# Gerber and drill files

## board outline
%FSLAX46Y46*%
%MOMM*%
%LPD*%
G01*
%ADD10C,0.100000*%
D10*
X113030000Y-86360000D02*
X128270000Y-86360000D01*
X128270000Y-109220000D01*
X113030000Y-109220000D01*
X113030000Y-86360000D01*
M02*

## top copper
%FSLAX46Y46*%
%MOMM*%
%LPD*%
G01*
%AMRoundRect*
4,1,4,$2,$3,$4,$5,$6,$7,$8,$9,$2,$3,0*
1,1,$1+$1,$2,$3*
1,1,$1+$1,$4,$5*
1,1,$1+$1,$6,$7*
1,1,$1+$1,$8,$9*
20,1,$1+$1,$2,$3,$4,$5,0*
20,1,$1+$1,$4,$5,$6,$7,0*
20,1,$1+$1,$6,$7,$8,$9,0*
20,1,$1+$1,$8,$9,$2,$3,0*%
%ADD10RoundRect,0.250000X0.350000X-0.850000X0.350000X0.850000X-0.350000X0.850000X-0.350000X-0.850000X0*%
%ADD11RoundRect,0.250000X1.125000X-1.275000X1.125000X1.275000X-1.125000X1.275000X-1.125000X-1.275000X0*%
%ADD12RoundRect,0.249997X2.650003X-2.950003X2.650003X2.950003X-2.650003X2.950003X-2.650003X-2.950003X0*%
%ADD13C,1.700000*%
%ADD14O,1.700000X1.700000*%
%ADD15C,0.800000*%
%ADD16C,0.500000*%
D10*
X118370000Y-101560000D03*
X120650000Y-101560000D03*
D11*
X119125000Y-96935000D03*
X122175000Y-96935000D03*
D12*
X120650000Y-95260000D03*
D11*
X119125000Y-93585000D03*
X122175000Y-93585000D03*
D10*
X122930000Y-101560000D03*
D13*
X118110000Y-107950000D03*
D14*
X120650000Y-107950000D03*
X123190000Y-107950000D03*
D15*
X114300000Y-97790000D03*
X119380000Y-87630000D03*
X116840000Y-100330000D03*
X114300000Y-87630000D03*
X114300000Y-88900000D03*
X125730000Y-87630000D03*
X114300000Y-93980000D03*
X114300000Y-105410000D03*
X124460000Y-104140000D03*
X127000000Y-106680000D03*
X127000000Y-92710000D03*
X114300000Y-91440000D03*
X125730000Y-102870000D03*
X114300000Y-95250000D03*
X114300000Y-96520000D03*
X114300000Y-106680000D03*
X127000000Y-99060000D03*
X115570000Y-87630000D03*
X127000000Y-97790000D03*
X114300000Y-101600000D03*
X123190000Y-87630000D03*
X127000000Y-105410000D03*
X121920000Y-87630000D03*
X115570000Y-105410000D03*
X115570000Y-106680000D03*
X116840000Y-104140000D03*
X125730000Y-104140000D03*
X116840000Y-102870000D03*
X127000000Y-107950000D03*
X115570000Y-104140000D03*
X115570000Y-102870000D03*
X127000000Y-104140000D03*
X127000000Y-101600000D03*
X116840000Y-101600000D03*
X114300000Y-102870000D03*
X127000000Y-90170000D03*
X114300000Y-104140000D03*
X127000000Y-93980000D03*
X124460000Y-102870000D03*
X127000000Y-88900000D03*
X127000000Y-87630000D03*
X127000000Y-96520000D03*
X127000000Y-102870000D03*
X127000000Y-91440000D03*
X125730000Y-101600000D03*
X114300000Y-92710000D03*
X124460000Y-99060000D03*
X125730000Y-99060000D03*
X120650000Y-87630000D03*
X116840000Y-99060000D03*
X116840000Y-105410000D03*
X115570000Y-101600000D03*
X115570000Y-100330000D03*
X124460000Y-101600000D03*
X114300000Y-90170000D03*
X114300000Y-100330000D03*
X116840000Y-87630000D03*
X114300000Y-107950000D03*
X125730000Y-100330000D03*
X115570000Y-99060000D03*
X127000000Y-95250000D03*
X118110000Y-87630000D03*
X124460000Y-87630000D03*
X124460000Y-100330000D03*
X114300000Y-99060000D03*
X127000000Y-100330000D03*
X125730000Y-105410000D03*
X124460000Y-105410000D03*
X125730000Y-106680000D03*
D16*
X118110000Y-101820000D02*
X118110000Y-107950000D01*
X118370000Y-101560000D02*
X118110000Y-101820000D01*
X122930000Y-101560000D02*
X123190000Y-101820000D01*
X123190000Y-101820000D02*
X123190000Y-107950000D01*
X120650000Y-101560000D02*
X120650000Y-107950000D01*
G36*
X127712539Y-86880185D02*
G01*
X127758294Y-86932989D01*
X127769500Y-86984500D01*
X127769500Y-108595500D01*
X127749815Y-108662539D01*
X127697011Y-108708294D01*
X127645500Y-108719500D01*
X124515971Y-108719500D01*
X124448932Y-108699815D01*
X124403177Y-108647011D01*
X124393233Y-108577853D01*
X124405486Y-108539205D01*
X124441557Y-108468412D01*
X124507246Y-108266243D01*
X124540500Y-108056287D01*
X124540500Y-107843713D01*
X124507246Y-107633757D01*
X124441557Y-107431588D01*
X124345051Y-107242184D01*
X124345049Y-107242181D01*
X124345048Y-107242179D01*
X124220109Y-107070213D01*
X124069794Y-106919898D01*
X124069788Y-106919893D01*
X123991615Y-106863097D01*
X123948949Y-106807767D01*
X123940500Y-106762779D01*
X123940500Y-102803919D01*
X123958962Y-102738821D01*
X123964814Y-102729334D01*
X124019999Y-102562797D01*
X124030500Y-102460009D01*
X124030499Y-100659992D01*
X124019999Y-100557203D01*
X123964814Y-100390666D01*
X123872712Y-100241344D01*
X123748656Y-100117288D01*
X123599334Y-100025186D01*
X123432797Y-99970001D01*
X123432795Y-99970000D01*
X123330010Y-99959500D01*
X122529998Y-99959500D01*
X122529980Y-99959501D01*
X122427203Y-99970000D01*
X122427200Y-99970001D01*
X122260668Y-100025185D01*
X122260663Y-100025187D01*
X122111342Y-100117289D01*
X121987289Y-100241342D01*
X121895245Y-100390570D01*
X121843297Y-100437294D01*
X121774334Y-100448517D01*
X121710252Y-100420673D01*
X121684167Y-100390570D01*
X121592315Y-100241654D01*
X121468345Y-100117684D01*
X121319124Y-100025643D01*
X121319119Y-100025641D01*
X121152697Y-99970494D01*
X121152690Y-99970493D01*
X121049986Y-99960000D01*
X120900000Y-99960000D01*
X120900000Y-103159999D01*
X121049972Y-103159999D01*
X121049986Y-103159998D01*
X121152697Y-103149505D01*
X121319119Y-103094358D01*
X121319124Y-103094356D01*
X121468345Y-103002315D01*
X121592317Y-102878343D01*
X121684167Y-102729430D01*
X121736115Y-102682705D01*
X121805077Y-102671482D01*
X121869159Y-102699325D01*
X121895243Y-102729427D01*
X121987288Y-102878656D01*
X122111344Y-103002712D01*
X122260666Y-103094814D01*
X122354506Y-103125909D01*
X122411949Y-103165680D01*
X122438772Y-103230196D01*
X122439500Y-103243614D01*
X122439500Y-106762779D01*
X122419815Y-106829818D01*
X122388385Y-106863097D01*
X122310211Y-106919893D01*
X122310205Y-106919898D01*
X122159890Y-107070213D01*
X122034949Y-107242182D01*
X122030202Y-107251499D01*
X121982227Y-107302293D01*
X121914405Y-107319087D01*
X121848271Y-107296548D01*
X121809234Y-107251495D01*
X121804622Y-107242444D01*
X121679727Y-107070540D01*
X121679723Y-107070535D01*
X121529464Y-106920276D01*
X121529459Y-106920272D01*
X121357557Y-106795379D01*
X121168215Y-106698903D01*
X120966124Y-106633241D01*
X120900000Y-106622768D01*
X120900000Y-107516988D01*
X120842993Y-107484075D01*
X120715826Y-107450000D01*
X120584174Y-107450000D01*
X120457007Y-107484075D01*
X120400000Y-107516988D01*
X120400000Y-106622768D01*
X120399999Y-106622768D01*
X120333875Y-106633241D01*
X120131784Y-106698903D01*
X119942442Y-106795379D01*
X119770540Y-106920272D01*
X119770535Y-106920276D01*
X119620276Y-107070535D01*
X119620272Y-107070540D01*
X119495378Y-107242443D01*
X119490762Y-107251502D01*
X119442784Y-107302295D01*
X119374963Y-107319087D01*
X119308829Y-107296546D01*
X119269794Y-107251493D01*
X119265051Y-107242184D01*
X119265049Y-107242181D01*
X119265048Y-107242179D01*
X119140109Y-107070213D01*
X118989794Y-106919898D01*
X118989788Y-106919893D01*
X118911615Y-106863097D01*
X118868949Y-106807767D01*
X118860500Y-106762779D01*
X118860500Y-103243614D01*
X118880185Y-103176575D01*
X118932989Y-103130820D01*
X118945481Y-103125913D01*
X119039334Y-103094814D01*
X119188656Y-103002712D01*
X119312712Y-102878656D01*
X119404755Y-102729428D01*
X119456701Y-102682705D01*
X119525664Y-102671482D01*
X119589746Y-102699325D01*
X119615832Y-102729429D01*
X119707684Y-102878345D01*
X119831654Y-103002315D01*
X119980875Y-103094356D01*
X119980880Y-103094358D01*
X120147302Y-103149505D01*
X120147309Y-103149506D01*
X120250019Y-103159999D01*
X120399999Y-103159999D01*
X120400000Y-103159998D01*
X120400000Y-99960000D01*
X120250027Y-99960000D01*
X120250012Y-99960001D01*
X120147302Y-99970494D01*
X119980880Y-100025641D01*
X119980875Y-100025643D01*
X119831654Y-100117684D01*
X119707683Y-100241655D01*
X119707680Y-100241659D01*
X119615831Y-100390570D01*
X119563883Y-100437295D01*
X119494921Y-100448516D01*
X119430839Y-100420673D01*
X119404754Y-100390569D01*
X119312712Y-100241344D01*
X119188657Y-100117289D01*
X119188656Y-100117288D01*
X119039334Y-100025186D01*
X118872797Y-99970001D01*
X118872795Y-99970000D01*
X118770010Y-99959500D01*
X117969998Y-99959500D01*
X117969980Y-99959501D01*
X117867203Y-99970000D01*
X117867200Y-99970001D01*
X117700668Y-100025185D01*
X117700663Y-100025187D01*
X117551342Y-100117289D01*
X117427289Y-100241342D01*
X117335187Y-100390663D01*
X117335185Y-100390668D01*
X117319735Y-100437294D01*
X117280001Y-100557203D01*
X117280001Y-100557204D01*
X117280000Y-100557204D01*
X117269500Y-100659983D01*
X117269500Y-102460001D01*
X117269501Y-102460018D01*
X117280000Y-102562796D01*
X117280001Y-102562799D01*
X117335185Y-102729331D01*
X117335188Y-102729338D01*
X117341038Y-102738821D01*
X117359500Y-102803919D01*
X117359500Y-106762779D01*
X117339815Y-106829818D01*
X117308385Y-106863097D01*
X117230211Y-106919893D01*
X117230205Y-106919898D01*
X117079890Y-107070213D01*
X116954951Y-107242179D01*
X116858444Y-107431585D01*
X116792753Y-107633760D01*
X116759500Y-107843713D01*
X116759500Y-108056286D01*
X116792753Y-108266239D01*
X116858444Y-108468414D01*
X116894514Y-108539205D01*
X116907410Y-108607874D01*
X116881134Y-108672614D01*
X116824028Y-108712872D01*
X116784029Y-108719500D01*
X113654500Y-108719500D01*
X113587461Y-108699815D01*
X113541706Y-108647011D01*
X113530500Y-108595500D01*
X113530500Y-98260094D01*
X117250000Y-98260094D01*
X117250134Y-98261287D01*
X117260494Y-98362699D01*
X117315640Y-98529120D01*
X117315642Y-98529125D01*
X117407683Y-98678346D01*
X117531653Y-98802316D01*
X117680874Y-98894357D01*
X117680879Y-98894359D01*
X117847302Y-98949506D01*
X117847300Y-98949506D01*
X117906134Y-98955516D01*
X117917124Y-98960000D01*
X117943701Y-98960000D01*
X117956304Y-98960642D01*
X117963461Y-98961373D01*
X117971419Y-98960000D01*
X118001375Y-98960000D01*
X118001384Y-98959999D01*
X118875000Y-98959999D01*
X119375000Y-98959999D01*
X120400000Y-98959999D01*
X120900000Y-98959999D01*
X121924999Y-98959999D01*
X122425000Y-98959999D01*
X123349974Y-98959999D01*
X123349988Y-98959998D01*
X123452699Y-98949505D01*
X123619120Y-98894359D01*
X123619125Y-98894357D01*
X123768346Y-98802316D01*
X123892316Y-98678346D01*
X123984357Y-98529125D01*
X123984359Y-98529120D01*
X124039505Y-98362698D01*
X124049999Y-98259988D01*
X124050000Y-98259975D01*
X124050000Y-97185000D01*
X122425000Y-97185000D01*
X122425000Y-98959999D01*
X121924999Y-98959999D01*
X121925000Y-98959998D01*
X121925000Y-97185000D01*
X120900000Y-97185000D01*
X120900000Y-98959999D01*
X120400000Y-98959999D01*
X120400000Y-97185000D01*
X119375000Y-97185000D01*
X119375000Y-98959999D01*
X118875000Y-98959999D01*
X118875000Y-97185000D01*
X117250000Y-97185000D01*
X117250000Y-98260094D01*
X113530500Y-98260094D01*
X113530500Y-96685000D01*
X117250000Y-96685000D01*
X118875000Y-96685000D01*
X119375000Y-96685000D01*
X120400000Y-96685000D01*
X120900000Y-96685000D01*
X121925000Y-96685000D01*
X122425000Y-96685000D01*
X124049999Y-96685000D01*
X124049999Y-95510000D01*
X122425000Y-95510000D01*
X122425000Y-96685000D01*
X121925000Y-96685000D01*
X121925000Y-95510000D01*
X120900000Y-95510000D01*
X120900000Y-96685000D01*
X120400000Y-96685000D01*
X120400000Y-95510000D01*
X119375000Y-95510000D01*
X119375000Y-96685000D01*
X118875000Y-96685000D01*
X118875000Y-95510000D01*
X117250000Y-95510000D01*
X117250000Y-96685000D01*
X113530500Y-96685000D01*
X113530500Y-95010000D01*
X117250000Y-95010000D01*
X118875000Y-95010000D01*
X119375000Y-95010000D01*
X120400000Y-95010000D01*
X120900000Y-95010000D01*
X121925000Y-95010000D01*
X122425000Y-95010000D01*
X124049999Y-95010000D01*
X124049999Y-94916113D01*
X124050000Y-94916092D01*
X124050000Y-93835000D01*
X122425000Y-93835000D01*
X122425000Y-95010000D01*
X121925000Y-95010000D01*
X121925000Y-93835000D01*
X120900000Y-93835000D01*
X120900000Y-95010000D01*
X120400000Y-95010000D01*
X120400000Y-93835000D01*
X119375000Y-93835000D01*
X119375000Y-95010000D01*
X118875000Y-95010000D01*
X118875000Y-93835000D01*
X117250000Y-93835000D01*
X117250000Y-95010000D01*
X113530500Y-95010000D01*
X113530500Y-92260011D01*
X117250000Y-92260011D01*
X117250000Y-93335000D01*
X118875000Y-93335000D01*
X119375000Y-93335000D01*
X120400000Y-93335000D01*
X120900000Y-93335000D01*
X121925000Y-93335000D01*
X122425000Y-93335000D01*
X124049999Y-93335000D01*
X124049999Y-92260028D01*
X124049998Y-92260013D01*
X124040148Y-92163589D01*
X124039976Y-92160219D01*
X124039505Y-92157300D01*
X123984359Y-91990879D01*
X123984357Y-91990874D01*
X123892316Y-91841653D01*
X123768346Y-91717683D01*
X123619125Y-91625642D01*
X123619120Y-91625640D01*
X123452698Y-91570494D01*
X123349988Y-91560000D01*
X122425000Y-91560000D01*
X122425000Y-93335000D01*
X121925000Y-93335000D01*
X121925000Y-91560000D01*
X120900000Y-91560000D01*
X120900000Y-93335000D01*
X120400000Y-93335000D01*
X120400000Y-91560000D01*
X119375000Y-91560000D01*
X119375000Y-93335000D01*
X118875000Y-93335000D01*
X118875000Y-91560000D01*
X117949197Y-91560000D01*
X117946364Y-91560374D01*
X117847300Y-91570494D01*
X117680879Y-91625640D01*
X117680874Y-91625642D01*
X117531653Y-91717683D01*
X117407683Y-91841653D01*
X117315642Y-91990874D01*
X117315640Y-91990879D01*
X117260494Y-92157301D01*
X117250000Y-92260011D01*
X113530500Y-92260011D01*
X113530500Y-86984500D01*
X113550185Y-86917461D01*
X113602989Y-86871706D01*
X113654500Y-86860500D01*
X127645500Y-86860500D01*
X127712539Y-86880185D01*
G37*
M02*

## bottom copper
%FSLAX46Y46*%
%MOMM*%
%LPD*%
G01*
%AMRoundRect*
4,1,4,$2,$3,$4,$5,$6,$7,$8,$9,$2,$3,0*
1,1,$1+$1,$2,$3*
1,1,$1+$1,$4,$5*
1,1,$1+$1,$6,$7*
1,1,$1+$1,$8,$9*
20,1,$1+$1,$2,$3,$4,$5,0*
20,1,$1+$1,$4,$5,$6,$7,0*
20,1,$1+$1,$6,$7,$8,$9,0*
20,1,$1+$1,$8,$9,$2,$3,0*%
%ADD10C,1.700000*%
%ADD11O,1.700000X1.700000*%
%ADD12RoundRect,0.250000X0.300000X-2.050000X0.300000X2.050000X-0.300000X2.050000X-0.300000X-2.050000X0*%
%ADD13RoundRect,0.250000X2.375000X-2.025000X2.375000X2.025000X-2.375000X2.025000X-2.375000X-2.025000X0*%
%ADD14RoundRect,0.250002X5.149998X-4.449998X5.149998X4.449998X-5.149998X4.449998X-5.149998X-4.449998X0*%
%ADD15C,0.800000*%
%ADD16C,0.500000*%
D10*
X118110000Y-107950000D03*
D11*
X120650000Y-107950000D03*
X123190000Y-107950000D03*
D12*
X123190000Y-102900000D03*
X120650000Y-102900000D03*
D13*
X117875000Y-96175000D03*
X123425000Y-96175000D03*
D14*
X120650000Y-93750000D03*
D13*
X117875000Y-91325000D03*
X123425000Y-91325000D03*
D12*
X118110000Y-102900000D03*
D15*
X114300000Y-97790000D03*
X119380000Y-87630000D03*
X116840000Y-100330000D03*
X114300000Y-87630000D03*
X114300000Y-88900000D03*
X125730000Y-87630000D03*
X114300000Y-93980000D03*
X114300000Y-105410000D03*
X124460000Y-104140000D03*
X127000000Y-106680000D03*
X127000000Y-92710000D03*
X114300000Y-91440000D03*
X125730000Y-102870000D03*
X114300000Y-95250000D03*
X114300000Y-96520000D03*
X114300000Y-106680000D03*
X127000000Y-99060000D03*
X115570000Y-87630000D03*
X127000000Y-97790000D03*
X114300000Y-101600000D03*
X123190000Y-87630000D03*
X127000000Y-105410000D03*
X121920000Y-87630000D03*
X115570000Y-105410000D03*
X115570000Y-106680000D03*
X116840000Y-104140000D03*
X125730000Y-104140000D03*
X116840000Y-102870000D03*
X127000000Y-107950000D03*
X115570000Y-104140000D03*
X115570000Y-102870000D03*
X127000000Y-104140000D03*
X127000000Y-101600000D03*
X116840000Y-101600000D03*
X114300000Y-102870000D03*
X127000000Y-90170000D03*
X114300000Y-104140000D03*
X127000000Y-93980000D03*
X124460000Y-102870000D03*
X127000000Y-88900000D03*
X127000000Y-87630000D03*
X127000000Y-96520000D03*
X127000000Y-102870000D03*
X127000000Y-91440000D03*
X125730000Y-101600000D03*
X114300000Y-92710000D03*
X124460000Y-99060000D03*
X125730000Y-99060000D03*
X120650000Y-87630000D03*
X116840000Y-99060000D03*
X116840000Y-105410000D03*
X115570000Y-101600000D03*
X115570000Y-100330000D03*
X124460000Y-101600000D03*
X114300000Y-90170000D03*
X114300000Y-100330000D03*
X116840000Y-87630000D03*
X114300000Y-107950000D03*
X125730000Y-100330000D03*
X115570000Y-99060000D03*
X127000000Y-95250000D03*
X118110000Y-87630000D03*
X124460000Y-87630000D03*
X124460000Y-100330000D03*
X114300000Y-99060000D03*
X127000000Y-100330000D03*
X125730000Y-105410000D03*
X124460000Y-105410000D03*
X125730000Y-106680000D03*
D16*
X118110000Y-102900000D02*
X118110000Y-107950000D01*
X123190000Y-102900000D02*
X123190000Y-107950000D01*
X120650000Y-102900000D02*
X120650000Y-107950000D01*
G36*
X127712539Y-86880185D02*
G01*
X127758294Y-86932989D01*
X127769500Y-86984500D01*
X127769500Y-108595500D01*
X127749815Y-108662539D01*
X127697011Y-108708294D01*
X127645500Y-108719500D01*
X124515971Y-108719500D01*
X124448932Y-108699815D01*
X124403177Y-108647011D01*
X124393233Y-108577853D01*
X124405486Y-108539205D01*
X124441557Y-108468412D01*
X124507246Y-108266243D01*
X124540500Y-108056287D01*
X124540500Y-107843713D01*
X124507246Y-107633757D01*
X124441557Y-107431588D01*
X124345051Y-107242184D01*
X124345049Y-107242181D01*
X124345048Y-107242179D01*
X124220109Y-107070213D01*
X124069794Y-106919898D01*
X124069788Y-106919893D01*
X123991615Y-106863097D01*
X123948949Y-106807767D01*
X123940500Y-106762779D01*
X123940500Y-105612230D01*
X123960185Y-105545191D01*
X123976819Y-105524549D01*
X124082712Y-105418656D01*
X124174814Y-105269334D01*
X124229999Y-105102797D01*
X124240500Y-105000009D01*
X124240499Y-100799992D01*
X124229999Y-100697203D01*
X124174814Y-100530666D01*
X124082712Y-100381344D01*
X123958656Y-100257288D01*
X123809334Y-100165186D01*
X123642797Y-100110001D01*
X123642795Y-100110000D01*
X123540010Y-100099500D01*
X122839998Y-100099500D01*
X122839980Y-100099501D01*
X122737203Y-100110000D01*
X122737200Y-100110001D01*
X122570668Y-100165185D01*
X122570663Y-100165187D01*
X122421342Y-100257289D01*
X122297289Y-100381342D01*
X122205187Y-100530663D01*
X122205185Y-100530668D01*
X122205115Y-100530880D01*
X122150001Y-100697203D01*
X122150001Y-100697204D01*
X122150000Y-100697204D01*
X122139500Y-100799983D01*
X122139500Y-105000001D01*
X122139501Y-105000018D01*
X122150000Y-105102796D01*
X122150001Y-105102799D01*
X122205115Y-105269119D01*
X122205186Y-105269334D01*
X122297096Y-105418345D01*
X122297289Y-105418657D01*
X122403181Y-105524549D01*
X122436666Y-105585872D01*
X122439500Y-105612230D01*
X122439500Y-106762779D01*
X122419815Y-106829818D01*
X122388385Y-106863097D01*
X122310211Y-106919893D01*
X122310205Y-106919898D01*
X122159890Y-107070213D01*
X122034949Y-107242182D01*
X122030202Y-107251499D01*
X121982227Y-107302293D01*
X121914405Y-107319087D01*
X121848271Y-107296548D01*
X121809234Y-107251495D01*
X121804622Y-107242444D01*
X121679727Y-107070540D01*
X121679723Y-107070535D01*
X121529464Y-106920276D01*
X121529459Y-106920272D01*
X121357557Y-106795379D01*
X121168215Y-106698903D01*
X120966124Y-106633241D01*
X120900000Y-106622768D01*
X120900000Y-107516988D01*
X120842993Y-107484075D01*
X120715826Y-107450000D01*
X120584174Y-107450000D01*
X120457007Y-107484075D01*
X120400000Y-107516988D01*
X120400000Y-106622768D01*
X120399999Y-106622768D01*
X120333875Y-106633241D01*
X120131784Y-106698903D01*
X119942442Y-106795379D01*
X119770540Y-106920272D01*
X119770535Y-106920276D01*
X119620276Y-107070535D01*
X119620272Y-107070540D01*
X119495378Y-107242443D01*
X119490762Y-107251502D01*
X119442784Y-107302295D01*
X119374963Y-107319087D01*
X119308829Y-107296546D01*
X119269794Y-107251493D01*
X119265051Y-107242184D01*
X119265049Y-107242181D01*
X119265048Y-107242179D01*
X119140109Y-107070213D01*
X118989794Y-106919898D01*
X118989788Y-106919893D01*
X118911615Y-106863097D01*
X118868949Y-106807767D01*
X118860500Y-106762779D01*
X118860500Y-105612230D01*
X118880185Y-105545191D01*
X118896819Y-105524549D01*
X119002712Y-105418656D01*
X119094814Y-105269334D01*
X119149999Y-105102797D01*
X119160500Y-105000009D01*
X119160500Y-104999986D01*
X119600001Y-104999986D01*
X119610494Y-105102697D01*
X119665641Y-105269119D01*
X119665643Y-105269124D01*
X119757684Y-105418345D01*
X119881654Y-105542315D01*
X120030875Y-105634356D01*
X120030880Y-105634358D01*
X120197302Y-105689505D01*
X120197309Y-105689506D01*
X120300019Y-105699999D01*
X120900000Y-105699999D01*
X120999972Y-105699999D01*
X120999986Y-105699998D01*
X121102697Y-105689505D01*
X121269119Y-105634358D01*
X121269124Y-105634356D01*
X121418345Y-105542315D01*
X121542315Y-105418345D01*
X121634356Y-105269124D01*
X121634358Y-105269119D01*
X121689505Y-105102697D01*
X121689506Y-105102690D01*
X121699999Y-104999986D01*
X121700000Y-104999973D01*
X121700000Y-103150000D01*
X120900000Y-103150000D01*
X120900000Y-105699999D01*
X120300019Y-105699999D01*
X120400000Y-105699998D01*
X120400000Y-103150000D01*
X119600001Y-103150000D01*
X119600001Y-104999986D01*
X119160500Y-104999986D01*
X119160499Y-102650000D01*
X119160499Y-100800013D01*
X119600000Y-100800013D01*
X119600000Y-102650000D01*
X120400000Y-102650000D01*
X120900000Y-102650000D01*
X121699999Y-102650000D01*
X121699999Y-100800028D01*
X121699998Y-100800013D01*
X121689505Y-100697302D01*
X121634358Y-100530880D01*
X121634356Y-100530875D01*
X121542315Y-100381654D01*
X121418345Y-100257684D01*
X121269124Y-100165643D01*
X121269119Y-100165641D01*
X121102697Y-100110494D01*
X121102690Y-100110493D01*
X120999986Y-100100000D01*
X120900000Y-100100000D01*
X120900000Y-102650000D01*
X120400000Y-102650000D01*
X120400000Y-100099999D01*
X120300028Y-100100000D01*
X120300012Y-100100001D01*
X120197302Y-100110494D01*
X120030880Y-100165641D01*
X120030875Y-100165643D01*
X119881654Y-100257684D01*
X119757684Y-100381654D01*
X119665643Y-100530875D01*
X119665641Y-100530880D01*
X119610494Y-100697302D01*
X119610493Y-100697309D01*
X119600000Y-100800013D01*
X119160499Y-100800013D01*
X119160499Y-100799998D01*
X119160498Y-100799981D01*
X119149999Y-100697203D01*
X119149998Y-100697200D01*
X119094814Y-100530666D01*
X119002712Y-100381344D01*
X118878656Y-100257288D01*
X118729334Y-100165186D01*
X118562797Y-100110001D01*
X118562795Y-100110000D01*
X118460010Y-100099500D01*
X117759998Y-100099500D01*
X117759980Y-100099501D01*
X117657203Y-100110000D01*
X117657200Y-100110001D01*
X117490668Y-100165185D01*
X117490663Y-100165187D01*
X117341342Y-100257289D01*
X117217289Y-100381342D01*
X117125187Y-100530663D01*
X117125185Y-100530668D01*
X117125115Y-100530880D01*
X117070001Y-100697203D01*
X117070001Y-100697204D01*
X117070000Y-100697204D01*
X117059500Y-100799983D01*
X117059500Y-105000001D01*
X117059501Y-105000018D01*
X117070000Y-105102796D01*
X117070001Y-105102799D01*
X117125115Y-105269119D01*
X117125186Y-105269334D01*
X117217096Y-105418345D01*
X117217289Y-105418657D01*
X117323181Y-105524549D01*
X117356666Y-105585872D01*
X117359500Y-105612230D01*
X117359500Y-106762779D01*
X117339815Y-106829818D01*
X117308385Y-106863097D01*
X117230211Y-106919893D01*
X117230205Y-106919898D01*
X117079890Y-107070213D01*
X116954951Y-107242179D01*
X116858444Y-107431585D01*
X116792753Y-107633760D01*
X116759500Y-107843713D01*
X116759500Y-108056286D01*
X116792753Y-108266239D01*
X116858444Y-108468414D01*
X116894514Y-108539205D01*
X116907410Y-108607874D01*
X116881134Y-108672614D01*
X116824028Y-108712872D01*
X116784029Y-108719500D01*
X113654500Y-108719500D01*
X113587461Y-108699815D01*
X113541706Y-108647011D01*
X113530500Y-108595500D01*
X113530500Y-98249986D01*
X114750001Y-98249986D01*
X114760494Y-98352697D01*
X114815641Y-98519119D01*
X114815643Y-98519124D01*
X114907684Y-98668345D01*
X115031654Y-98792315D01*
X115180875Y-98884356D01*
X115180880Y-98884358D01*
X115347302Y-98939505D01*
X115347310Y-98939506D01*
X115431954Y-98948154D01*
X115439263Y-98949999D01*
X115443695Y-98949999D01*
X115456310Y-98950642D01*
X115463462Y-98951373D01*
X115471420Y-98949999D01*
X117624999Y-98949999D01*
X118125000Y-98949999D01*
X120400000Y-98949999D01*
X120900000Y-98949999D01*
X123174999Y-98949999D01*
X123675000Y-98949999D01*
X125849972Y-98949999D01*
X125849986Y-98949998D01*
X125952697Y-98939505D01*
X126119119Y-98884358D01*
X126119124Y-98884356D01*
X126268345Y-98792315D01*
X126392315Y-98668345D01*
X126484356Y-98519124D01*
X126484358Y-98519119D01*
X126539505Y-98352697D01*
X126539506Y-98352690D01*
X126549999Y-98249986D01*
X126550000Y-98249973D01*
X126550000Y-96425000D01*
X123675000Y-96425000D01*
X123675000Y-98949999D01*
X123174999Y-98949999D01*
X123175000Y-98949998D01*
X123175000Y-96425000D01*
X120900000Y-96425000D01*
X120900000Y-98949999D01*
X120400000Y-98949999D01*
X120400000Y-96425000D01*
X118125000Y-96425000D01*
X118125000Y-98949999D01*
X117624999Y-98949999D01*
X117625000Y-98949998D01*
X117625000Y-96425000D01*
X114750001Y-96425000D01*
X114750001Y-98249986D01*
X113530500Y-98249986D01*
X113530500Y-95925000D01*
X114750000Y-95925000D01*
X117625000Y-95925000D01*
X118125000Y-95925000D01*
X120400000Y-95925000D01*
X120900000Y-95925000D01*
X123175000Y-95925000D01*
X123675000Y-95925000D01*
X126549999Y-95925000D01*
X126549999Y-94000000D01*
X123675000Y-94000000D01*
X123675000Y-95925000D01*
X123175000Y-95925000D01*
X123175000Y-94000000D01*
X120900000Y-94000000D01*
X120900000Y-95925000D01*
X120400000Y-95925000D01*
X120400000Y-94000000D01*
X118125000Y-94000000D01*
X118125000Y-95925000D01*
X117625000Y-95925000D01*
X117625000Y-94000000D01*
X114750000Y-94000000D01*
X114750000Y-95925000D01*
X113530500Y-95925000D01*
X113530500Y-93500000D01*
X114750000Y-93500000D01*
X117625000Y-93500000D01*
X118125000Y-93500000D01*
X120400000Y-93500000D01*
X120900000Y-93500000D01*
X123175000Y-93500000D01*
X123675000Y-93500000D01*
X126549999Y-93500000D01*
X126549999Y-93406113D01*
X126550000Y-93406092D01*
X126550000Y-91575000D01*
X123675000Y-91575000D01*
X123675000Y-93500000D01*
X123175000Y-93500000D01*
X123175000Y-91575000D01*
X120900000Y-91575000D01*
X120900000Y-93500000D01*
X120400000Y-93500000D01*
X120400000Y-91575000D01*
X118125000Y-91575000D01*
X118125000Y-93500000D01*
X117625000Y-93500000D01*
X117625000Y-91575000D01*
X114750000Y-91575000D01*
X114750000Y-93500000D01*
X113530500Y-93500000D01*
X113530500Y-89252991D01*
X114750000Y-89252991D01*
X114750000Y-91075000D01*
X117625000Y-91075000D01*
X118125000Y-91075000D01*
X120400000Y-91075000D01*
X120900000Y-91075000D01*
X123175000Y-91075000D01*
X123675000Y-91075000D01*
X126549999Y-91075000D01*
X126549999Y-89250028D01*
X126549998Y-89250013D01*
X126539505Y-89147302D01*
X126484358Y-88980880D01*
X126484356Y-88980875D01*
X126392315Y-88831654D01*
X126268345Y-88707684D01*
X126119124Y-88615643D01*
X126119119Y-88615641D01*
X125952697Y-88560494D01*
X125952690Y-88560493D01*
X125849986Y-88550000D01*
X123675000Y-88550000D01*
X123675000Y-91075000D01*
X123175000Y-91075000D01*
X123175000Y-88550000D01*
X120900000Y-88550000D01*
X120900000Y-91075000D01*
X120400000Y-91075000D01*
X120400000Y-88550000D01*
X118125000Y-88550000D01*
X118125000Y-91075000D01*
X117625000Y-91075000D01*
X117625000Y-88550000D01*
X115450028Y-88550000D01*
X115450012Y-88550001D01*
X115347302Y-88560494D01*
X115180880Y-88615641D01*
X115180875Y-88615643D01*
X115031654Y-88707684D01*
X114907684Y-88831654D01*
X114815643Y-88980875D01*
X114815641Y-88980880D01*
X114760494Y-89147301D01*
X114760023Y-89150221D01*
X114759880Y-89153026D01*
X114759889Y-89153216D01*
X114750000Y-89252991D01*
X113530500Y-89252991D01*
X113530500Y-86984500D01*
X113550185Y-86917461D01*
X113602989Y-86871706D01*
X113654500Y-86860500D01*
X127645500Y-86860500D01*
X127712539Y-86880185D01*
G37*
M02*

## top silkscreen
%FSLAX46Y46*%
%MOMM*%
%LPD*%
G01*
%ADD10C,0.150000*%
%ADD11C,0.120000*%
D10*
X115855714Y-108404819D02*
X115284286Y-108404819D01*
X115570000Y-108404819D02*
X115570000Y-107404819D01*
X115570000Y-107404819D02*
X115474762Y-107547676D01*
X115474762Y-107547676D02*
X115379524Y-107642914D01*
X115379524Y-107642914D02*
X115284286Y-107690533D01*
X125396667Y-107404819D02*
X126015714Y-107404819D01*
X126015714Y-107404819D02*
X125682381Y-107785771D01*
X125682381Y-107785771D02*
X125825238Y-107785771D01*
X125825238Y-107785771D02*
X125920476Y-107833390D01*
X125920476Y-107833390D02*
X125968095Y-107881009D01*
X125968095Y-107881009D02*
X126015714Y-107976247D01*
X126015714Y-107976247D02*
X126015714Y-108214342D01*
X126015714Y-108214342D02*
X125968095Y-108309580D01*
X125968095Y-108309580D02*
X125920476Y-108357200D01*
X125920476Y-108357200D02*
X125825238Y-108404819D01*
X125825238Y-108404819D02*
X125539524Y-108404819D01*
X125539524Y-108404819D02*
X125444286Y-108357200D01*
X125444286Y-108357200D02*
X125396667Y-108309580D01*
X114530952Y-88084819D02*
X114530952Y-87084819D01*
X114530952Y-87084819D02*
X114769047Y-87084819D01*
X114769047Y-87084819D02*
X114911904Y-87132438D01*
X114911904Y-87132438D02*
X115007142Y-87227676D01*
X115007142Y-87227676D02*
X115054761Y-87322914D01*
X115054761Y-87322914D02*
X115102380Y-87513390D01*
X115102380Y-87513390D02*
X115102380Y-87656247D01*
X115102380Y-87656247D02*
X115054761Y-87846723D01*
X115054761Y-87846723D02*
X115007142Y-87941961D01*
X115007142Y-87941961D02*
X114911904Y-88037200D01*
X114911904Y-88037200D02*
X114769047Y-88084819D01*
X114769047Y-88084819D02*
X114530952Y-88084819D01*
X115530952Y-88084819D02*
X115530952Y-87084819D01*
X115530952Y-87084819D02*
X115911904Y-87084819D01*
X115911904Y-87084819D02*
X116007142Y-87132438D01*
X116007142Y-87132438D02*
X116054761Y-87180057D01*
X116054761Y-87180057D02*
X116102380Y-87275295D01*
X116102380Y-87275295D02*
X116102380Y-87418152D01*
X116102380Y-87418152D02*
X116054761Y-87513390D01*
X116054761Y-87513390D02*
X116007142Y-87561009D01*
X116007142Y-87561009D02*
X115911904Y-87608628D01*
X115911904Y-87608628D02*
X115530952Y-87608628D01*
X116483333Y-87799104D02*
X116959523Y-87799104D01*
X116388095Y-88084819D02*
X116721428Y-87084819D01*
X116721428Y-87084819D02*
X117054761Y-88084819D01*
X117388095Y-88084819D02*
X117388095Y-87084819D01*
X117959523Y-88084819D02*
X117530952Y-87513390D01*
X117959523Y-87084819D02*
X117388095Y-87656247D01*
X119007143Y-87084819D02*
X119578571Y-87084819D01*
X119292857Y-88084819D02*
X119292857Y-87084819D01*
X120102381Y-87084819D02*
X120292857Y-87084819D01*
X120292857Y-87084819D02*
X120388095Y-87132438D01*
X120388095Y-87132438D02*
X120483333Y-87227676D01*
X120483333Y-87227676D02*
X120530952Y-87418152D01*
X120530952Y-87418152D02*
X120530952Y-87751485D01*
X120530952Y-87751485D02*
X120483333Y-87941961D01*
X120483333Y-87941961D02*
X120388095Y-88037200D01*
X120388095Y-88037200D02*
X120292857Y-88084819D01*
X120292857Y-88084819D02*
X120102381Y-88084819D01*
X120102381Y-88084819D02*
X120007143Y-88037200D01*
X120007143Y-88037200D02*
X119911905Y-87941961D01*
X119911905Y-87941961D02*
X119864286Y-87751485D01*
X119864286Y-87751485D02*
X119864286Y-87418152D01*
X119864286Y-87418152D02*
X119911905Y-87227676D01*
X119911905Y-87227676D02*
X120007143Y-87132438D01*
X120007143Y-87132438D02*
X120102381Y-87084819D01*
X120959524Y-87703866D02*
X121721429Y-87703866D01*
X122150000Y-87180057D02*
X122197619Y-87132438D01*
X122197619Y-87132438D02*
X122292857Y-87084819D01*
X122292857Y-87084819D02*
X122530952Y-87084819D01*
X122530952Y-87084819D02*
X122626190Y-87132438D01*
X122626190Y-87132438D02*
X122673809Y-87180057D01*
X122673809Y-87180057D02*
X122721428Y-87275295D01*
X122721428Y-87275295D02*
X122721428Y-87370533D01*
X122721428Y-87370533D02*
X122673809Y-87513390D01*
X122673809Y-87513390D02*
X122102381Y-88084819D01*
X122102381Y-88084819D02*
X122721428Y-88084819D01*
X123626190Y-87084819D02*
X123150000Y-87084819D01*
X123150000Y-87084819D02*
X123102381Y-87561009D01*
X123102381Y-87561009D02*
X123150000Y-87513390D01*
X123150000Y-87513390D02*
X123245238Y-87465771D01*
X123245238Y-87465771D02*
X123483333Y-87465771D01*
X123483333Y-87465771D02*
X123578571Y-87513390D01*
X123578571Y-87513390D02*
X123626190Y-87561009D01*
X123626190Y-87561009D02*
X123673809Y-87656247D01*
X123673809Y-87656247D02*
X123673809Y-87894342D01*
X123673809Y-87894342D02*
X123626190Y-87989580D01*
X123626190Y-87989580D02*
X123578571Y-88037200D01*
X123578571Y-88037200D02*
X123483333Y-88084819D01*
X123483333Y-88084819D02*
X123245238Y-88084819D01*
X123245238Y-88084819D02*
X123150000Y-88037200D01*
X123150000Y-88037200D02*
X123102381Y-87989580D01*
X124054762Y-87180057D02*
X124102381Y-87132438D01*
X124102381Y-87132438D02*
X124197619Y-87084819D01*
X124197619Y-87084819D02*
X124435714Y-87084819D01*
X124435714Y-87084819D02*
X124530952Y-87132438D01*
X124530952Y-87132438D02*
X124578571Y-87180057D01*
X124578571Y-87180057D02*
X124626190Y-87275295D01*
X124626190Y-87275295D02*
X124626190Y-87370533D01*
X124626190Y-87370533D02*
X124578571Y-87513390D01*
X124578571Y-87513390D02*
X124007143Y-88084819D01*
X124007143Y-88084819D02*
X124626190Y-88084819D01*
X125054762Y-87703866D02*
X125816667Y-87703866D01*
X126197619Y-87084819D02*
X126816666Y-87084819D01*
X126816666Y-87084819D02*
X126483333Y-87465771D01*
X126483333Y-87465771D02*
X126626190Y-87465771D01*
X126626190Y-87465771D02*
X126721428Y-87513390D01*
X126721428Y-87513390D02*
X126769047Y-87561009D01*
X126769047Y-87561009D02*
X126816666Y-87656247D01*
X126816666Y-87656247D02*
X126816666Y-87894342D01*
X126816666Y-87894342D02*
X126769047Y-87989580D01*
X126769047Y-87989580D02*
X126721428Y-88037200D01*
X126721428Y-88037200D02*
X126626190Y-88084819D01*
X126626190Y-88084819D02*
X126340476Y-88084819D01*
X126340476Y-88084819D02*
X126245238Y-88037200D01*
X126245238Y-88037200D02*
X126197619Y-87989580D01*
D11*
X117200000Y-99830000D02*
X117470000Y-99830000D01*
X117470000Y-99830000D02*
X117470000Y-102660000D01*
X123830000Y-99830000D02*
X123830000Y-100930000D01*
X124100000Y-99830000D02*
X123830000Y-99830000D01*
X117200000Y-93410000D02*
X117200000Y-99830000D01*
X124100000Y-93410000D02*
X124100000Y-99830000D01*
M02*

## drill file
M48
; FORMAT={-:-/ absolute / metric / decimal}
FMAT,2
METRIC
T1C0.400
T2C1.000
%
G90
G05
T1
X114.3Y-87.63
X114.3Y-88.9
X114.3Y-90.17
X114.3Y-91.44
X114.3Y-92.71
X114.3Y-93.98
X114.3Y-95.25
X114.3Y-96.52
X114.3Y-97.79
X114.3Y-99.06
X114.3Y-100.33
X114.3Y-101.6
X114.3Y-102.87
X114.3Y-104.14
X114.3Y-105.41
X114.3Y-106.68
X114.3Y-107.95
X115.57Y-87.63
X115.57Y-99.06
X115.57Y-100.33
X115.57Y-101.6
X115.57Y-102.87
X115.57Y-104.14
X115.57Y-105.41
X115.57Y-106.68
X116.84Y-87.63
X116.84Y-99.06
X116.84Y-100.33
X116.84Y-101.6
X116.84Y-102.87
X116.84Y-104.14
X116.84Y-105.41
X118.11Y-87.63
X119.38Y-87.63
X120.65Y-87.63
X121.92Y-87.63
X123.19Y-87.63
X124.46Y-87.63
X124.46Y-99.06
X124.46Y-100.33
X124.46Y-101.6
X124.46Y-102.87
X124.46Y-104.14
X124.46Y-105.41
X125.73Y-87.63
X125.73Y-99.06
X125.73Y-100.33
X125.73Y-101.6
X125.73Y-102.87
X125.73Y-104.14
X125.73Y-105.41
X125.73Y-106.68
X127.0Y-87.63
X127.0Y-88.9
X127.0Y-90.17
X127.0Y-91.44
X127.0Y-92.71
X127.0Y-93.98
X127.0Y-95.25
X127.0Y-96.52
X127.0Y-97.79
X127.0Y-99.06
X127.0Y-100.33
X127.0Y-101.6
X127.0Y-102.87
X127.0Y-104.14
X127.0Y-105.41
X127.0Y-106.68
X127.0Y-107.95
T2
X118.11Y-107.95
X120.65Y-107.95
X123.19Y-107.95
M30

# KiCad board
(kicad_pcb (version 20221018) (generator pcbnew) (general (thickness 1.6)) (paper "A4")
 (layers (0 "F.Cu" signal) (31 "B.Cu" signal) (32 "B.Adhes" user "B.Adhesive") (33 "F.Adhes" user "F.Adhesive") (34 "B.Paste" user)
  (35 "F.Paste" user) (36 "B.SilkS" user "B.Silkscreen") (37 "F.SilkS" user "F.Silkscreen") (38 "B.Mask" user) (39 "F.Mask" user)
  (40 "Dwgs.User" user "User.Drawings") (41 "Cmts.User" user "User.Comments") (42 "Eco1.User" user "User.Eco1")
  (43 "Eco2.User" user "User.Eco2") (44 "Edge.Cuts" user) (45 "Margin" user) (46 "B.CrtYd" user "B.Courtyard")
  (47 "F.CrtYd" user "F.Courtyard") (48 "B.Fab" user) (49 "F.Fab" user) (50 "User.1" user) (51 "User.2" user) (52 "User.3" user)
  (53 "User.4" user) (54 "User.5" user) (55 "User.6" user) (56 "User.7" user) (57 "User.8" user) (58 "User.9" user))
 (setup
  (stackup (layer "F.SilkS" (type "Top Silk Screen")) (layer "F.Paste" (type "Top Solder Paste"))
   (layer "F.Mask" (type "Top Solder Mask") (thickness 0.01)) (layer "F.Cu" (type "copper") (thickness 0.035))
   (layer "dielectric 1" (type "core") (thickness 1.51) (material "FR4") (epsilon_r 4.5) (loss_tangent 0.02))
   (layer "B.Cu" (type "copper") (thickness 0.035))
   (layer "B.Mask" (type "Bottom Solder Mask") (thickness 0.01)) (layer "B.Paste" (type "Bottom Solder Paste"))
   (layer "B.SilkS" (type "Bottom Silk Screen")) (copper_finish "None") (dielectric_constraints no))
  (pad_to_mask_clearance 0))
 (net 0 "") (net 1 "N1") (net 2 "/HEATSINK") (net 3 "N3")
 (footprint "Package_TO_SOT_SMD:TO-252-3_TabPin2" (layer "F.Cu") (at 120.65 96.52 90)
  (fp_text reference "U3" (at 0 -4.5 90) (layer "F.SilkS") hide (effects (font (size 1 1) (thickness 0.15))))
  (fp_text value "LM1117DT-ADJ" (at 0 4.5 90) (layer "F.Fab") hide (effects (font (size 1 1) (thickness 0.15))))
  (fp_line (start -3.31 -3.45) (end -3.31 -3.18) (stroke (width 0.12) (type solid)) (layer "F.SilkS"))
  (fp_line (start -3.31 -3.18) (end -6.14 -3.18) (stroke (width 0.12) (type solid)) (layer "F.SilkS"))
  (fp_line (start -3.31 3.18) (end -4.41 3.18) (stroke (width 0.12) (type solid)) (layer "F.SilkS"))
  (fp_line (start -3.31 3.45) (end -3.31 3.18) (stroke (width 0.12) (type solid)) (layer "F.SilkS"))
  (fp_line (start 3.11 -3.45) (end -3.31 -3.45) (stroke (width 0.12) (type solid)) (layer "F.SilkS"))
  (fp_line (start 3.11 3.45) (end -3.31 3.45) (stroke (width 0.12) (type solid)) (layer "F.SilkS"))
  (pad "1" smd roundrect (at -5.04 -2.28 90) (size 2.2 1.2) (layers "F.Cu" "F.Paste" "F.Mask") (roundrect_rratio 0.208333) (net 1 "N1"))
  (pad "2" smd roundrect (at -5.04 0 90) (size 2.2 1.2) (layers "F.Cu" "F.Paste" "F.Mask") (roundrect_rratio 0.208333) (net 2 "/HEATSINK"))
  (pad "2" smd roundrect (at -0.415 -1.525 90) (size 3.05 2.75) (layers "F.Cu" "F.Paste") (roundrect_rratio 0.090909) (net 2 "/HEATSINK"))
  (pad "2" smd roundrect (at -0.415 1.525 90) (size 3.05 2.75) (layers "F.Cu" "F.Paste") (roundrect_rratio 0.090909) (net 2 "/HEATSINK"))
  (pad "2" smd roundrect (at 1.26 0 90) (size 6.4 5.8) (layers "F.Cu" "F.Mask") (roundrect_rratio 0.043103) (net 2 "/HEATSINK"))
  (pad "2" smd roundrect (at 2.935 -1.525 90) (size 3.05 2.75) (layers "F.Cu" "F.Paste") (roundrect_rratio 0.090909) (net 2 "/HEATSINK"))
  (pad "2" smd roundrect (at 2.935 1.525 90) (size 3.05 2.75) (layers "F.Cu" "F.Paste") (roundrect_rratio 0.090909) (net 2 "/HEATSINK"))
  (pad "3" smd roundrect (at -5.04 2.28 90) (size 2.2 1.2) (layers "F.Cu" "F.Paste" "F.Mask") (roundrect_rratio 0.208333) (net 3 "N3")))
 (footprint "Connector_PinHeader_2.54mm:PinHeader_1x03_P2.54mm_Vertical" (layer "F.Cu") (at 118.11 107.95 90)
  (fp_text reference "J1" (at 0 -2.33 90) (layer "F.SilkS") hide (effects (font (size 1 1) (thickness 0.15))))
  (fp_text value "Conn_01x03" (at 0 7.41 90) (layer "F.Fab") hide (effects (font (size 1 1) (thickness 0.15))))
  (pad "1" thru_hole circle (at 0 0 90) (size 1.7 1.7) (drill 1) (layers "*.Cu" "*.Mask") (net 1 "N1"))
  (pad "2" thru_hole oval (at 0 2.54 90) (size 1.7 1.7) (drill 1) (layers "*.Cu" "*.Mask") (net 2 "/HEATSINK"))
  (pad "3" thru_hole oval (at 0 5.08 90) (size 1.7 1.7) (drill 1) (layers "*.Cu" "*.Mask") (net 3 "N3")))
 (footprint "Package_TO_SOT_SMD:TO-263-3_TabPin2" (layer "B.Cu") (at 120.65 95.25 90)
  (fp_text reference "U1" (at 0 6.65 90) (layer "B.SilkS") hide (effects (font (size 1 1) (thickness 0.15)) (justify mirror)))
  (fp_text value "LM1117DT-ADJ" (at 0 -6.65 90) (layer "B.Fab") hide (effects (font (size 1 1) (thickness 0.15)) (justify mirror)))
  (pad "1" smd roundrect (at -7.65 2.54 90) (size 4.6 1.1) (layers "B.Cu" "B.Paste" "B.Mask") (roundrect_rratio 0.227273) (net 3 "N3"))
  (pad "2" smd roundrect (at -7.65 0 90) (size 4.6 1.1) (layers "B.Cu" "B.Paste" "B.Mask") (roundrect_rratio 0.227273) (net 2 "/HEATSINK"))
  (pad "2" smd roundrect (at -0.925 -2.775 90) (size 4.55 5.25) (layers "B.Cu" "B.Paste") (roundrect_rratio 0.054945) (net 2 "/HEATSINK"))
  (pad "2" smd roundrect (at -0.925 2.775 90) (size 4.55 5.25) (layers "B.Cu" "B.Paste") (roundrect_rratio 0.054945) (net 2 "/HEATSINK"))
  (pad "2" smd roundrect (at 1.5 0 90) (size 9.4 10.8) (layers "B.Cu" "B.Mask") (roundrect_rratio 0.026596) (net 2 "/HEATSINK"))
  (pad "2" smd roundrect (at 3.925 -2.775 90) (size 4.55 5.25) (layers "B.Cu" "B.Paste") (roundrect_rratio 0.054945) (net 2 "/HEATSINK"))
  (pad "2" smd roundrect (at 3.925 2.775 90) (size 4.55 5.25) (layers "B.Cu" "B.Paste") (roundrect_rratio 0.054945) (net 2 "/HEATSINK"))
  (pad "3" smd roundrect (at -7.65 -2.54 90) (size 4.6 1.1) (layers "B.Cu" "B.Paste" "B.Mask") (roundrect_rratio 0.227273) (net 1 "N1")))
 (gr_rect (start 113.03 86.36) (end 128.27 109.22) (stroke (width 0.1) (type default)) (fill none) (layer "Edge.Cuts"))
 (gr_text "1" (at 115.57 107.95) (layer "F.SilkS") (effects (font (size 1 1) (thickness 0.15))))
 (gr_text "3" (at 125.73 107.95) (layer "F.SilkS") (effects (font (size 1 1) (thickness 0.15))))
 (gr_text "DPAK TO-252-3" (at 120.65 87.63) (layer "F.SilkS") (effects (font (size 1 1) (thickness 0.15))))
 (segment (start 118.11 101.82) (end 118.11 107.95) (width 0.5) (layer "F.Cu") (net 1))
 (segment (start 118.37 101.56) (end 118.11 101.82) (width 0.5) (layer "F.Cu") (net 1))
 (segment (start 118.11 102.9) (end 118.11 107.95) (width 0.5) (layer "B.Cu") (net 1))
 (segment (start 122.93 101.56) (end 123.19 101.82) (width 0.5) (layer "F.Cu") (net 3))
 (segment (start 123.19 101.82) (end 123.19 107.95) (width 0.5) (layer "F.Cu") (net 3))
 (segment (start 123.19 102.9) (end 123.19 107.95) (width 0.5) (layer "B.Cu") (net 3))
 (segment (start 120.65 101.56) (end 120.65 107.95) (width 0.5) (layer "F.Cu") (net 2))
 (via (at 114.3 97.79) (size 0.8) (drill 0.4) (layers "F.Cu" "B.Cu") (free) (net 2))
 (via (at 119.38 87.63) (size 0.8) (drill 0.4) (layers "F.Cu" "B.Cu") (free) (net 2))
 (via (at 116.84 100.33) (size 0.8) (drill 0.4) (layers "F.Cu" "B.Cu") (free) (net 2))
 (via (at 114.3 87.63) (size 0.8) (drill 0.4) (layers "F.Cu" "B.Cu") (free) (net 2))
 (via (at 114.3 88.9) (size 0.8) (drill 0.4) (layers "F.Cu" "B.Cu") (free) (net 2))
 (via (at 125.73 87.63) (size 0.8) (drill 0.4) (layers "F.Cu" "B.Cu") (free) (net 2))
 (via (at 114.3 93.98) (size 0.8) (drill 0.4) (layers "F.Cu" "B.Cu") (free) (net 2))
 (via (at 114.3 105.41) (size 0.8) (drill 0.4) (layers "F.Cu" "B.Cu") (free) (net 2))
 (via (at 124.46 104.14) (size 0.8) (drill 0.4) (layers "F.Cu" "B.Cu") (free) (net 2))
 (via (at 127 106.68) (size 0.8) (drill 0.4) (layers "F.Cu" "B.Cu") (free) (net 2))
 (via (at 127 92.71) (size 0.8) (drill 0.4) (layers "F.Cu" "B.Cu") (free) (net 2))
 (via (at 114.3 91.44) (size 0.8) (drill 0.4) (layers "F.Cu" "B.Cu") (free) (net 2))
 (via (at 125.73 102.87) (size 0.8) (drill 0.4) (layers "F.Cu" "B.Cu") (free) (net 2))
 (via (at 114.3 95.25) (size 0.8) (drill 0.4) (layers "F.Cu" "B.Cu") (free) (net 2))
 (via (at 114.3 96.52) (size 0.8) (drill 0.4) (layers "F.Cu" "B.Cu") (free) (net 2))
 (via (at 114.3 106.68) (size 0.8) (drill 0.4) (layers "F.Cu" "B.Cu") (free) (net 2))
 (via (at 127 99.06) (size 0.8) (drill 0.4) (layers "F.Cu" "B.Cu") (free) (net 2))
 (via (at 115.57 87.63) (size 0.8) (drill 0.4) (layers "F.Cu" "B.Cu") (free) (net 2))
 (via (at 127 97.79) (size 0.8) (drill 0.4) (layers "F.Cu" "B.Cu") (free) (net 2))
 (via (at 114.3 101.6) (size 0.8) (drill 0.4) (layers "F.Cu" "B.Cu") (free) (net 2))
 (via (at 123.19 87.63) (size 0.8) (drill 0.4) (layers "F.Cu" "B.Cu") (free) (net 2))
 (via (at 127 105.41) (size 0.8) (drill 0.4) (layers "F.Cu" "B.Cu") (free) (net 2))
 (via (at 121.92 87.63) (size 0.8) (drill 0.4) (layers "F.Cu" "B.Cu") (free) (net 2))
 (via (at 115.57 105.41) (size 0.8) (drill 0.4) (layers "F.Cu" "B.Cu") (free) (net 2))
 (via (at 115.57 106.68) (size 0.8) (drill 0.4) (layers "F.Cu" "B.Cu") (free) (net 2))
 (via (at 116.84 104.14) (size 0.8) (drill 0.4) (layers "F.Cu" "B.Cu") (free) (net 2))
 (via (at 125.73 104.14) (size 0.8) (drill 0.4) (layers "F.Cu" "B.Cu") (free) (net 2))
 (via (at 116.84 102.87) (size 0.8) (drill 0.4) (layers "F.Cu" "B.Cu") (free) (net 2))
 (via (at 127 107.95) (size 0.8) (drill 0.4) (layers "F.Cu" "B.Cu") (free) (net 2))
 (via (at 115.57 104.14) (size 0.8) (drill 0.4) (layers "F.Cu" "B.Cu") (free) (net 2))
 (via (at 115.57 102.87) (size 0.8) (drill 0.4) (layers "F.Cu" "B.Cu") (free) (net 2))
 (via (at 127 104.14) (size 0.8) (drill 0.4) (layers "F.Cu" "B.Cu") (free) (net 2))
 (via (at 127 101.6) (size 0.8) (drill 0.4) (layers "F.Cu" "B.Cu") (free) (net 2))
 (via (at 116.84 101.6) (size 0.8) (drill 0.4) (layers "F.Cu" "B.Cu") (free) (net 2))
 (via (at 114.3 102.87) (size 0.8) (drill 0.4) (layers "F.Cu" "B.Cu") (free) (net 2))
 (via (at 127 90.17) (size 0.8) (drill 0.4) (layers "F.Cu" "B.Cu") (free) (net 2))
 (via (at 114.3 104.14) (size 0.8) (drill 0.4) (layers "F.Cu" "B.Cu") (free) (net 2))
 (via (at 127 93.98) (size 0.8) (drill 0.4) (layers "F.Cu" "B.Cu") (free) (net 2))
 (via (at 124.46 102.87) (size 0.8) (drill 0.4) (layers "F.Cu" "B.Cu") (free) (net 2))
 (via (at 127 88.9) (size 0.8) (drill 0.4) (layers "F.Cu" "B.Cu") (free) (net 2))
 (via (at 127 87.63) (size 0.8) (drill 0.4) (layers "F.Cu" "B.Cu") (free) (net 2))
 (via (at 127 96.52) (size 0.8) (drill 0.4) (layers "F.Cu" "B.Cu") (free) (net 2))
 (via (at 127 102.87) (size 0.8) (drill 0.4) (layers "F.Cu" "B.Cu") (free) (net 2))
 (via (at 127 91.44) (size 0.8) (drill 0.4) (layers "F.Cu" "B.Cu") (free) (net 2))
 (via (at 125.73 101.6) (size 0.8) (drill 0.4) (layers "F.Cu" "B.Cu") (free) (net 2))
 (via (at 114.3 92.71) (size 0.8) (drill 0.4) (layers "F.Cu" "B.Cu") (free) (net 2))
 (via (at 124.46 99.06) (size 0.8) (drill 0.4) (layers "F.Cu" "B.Cu") (free) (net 2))
 (via (at 125.73 99.06) (size 0.8) (drill 0.4) (layers "F.Cu" "B.Cu") (free) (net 2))
 (via (at 120.65 87.63) (size 0.8) (drill 0.4) (layers "F.Cu" "B.Cu") (free) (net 2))
 (via (at 116.84 99.06) (size 0.8) (drill 0.4) (layers "F.Cu" "B.Cu") (free) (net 2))
 (via (at 116.84 105.41) (size 0.8) (drill 0.4) (layers "F.Cu" "B.Cu") (free) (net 2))
 (via (at 115.57 101.6) (size 0.8) (drill 0.4) (layers "F.Cu" "B.Cu") (free) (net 2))
 (via (at 115.57 100.33) (size 0.8) (drill 0.4) (layers "F.Cu" "B.Cu") (free) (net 2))
 (via (at 124.46 101.6) (size 0.8) (drill 0.4) (layers "F.Cu" "B.Cu") (free) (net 2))
 (via (at 114.3 90.17) (size 0.8) (drill 0.4) (layers "F.Cu" "B.Cu") (free) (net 2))
 (via (at 114.3 100.33) (size 0.8) (drill 0.4) (layers "F.Cu" "B.Cu") (free) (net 2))
 (via (at 116.84 87.63) (size 0.8) (drill 0.4) (layers "F.Cu" "B.Cu") (free) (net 2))
 (via (at 114.3 107.95) (size 0.8) (drill 0.4) (layers "F.Cu" "B.Cu") (free) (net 2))
 (via (at 125.73 100.33) (size 0.8) (drill 0.4) (layers "F.Cu" "B.Cu") (free) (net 2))
 (via (at 115.57 99.06) (size 0.8) (drill 0.4) (layers "F.Cu" "B.Cu") (free) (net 2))
 (via (at 127 95.25) (size 0.8) (drill 0.4) (layers "F.Cu" "B.Cu") (free) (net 2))
 (via (at 118.11 87.63) (size 0.8) (drill 0.4) (layers "F.Cu" "B.Cu") (free) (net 2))
 (via (at 124.46 87.63) (size 0.8) (drill 0.4) (layers "F.Cu" "B.Cu") (free) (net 2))
 (via (at 124.46 100.33) (size 0.8) (drill 0.4) (layers "F.Cu" "B.Cu") (free) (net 2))
 (via (at 114.3 99.06) (size 0.8) (drill 0.4) (layers "F.Cu" "B.Cu") (free) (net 2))
 (via (at 127 100.33) (size 0.8) (drill 0.4) (layers "F.Cu" "B.Cu") (free) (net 2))
 (via (at 125.73 105.41) (size 0.8) (drill 0.4) (layers "F.Cu" "B.Cu") (free) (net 2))
 (via (at 124.46 105.41) (size 0.8) (drill 0.4) (layers "F.Cu" "B.Cu") (free) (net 2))
 (via (at 125.73 106.68) (size 0.8) (drill 0.4) (layers "F.Cu" "B.Cu") (free) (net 2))
 (segment (start 120.65 102.9) (end 120.65 107.95) (width 0.5) (layer "B.Cu") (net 2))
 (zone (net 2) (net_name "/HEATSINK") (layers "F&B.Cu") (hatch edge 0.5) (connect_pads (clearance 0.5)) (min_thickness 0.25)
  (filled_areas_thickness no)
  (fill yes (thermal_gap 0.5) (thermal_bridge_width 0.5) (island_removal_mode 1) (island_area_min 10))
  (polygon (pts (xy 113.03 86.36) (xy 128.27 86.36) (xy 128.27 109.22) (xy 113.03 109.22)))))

